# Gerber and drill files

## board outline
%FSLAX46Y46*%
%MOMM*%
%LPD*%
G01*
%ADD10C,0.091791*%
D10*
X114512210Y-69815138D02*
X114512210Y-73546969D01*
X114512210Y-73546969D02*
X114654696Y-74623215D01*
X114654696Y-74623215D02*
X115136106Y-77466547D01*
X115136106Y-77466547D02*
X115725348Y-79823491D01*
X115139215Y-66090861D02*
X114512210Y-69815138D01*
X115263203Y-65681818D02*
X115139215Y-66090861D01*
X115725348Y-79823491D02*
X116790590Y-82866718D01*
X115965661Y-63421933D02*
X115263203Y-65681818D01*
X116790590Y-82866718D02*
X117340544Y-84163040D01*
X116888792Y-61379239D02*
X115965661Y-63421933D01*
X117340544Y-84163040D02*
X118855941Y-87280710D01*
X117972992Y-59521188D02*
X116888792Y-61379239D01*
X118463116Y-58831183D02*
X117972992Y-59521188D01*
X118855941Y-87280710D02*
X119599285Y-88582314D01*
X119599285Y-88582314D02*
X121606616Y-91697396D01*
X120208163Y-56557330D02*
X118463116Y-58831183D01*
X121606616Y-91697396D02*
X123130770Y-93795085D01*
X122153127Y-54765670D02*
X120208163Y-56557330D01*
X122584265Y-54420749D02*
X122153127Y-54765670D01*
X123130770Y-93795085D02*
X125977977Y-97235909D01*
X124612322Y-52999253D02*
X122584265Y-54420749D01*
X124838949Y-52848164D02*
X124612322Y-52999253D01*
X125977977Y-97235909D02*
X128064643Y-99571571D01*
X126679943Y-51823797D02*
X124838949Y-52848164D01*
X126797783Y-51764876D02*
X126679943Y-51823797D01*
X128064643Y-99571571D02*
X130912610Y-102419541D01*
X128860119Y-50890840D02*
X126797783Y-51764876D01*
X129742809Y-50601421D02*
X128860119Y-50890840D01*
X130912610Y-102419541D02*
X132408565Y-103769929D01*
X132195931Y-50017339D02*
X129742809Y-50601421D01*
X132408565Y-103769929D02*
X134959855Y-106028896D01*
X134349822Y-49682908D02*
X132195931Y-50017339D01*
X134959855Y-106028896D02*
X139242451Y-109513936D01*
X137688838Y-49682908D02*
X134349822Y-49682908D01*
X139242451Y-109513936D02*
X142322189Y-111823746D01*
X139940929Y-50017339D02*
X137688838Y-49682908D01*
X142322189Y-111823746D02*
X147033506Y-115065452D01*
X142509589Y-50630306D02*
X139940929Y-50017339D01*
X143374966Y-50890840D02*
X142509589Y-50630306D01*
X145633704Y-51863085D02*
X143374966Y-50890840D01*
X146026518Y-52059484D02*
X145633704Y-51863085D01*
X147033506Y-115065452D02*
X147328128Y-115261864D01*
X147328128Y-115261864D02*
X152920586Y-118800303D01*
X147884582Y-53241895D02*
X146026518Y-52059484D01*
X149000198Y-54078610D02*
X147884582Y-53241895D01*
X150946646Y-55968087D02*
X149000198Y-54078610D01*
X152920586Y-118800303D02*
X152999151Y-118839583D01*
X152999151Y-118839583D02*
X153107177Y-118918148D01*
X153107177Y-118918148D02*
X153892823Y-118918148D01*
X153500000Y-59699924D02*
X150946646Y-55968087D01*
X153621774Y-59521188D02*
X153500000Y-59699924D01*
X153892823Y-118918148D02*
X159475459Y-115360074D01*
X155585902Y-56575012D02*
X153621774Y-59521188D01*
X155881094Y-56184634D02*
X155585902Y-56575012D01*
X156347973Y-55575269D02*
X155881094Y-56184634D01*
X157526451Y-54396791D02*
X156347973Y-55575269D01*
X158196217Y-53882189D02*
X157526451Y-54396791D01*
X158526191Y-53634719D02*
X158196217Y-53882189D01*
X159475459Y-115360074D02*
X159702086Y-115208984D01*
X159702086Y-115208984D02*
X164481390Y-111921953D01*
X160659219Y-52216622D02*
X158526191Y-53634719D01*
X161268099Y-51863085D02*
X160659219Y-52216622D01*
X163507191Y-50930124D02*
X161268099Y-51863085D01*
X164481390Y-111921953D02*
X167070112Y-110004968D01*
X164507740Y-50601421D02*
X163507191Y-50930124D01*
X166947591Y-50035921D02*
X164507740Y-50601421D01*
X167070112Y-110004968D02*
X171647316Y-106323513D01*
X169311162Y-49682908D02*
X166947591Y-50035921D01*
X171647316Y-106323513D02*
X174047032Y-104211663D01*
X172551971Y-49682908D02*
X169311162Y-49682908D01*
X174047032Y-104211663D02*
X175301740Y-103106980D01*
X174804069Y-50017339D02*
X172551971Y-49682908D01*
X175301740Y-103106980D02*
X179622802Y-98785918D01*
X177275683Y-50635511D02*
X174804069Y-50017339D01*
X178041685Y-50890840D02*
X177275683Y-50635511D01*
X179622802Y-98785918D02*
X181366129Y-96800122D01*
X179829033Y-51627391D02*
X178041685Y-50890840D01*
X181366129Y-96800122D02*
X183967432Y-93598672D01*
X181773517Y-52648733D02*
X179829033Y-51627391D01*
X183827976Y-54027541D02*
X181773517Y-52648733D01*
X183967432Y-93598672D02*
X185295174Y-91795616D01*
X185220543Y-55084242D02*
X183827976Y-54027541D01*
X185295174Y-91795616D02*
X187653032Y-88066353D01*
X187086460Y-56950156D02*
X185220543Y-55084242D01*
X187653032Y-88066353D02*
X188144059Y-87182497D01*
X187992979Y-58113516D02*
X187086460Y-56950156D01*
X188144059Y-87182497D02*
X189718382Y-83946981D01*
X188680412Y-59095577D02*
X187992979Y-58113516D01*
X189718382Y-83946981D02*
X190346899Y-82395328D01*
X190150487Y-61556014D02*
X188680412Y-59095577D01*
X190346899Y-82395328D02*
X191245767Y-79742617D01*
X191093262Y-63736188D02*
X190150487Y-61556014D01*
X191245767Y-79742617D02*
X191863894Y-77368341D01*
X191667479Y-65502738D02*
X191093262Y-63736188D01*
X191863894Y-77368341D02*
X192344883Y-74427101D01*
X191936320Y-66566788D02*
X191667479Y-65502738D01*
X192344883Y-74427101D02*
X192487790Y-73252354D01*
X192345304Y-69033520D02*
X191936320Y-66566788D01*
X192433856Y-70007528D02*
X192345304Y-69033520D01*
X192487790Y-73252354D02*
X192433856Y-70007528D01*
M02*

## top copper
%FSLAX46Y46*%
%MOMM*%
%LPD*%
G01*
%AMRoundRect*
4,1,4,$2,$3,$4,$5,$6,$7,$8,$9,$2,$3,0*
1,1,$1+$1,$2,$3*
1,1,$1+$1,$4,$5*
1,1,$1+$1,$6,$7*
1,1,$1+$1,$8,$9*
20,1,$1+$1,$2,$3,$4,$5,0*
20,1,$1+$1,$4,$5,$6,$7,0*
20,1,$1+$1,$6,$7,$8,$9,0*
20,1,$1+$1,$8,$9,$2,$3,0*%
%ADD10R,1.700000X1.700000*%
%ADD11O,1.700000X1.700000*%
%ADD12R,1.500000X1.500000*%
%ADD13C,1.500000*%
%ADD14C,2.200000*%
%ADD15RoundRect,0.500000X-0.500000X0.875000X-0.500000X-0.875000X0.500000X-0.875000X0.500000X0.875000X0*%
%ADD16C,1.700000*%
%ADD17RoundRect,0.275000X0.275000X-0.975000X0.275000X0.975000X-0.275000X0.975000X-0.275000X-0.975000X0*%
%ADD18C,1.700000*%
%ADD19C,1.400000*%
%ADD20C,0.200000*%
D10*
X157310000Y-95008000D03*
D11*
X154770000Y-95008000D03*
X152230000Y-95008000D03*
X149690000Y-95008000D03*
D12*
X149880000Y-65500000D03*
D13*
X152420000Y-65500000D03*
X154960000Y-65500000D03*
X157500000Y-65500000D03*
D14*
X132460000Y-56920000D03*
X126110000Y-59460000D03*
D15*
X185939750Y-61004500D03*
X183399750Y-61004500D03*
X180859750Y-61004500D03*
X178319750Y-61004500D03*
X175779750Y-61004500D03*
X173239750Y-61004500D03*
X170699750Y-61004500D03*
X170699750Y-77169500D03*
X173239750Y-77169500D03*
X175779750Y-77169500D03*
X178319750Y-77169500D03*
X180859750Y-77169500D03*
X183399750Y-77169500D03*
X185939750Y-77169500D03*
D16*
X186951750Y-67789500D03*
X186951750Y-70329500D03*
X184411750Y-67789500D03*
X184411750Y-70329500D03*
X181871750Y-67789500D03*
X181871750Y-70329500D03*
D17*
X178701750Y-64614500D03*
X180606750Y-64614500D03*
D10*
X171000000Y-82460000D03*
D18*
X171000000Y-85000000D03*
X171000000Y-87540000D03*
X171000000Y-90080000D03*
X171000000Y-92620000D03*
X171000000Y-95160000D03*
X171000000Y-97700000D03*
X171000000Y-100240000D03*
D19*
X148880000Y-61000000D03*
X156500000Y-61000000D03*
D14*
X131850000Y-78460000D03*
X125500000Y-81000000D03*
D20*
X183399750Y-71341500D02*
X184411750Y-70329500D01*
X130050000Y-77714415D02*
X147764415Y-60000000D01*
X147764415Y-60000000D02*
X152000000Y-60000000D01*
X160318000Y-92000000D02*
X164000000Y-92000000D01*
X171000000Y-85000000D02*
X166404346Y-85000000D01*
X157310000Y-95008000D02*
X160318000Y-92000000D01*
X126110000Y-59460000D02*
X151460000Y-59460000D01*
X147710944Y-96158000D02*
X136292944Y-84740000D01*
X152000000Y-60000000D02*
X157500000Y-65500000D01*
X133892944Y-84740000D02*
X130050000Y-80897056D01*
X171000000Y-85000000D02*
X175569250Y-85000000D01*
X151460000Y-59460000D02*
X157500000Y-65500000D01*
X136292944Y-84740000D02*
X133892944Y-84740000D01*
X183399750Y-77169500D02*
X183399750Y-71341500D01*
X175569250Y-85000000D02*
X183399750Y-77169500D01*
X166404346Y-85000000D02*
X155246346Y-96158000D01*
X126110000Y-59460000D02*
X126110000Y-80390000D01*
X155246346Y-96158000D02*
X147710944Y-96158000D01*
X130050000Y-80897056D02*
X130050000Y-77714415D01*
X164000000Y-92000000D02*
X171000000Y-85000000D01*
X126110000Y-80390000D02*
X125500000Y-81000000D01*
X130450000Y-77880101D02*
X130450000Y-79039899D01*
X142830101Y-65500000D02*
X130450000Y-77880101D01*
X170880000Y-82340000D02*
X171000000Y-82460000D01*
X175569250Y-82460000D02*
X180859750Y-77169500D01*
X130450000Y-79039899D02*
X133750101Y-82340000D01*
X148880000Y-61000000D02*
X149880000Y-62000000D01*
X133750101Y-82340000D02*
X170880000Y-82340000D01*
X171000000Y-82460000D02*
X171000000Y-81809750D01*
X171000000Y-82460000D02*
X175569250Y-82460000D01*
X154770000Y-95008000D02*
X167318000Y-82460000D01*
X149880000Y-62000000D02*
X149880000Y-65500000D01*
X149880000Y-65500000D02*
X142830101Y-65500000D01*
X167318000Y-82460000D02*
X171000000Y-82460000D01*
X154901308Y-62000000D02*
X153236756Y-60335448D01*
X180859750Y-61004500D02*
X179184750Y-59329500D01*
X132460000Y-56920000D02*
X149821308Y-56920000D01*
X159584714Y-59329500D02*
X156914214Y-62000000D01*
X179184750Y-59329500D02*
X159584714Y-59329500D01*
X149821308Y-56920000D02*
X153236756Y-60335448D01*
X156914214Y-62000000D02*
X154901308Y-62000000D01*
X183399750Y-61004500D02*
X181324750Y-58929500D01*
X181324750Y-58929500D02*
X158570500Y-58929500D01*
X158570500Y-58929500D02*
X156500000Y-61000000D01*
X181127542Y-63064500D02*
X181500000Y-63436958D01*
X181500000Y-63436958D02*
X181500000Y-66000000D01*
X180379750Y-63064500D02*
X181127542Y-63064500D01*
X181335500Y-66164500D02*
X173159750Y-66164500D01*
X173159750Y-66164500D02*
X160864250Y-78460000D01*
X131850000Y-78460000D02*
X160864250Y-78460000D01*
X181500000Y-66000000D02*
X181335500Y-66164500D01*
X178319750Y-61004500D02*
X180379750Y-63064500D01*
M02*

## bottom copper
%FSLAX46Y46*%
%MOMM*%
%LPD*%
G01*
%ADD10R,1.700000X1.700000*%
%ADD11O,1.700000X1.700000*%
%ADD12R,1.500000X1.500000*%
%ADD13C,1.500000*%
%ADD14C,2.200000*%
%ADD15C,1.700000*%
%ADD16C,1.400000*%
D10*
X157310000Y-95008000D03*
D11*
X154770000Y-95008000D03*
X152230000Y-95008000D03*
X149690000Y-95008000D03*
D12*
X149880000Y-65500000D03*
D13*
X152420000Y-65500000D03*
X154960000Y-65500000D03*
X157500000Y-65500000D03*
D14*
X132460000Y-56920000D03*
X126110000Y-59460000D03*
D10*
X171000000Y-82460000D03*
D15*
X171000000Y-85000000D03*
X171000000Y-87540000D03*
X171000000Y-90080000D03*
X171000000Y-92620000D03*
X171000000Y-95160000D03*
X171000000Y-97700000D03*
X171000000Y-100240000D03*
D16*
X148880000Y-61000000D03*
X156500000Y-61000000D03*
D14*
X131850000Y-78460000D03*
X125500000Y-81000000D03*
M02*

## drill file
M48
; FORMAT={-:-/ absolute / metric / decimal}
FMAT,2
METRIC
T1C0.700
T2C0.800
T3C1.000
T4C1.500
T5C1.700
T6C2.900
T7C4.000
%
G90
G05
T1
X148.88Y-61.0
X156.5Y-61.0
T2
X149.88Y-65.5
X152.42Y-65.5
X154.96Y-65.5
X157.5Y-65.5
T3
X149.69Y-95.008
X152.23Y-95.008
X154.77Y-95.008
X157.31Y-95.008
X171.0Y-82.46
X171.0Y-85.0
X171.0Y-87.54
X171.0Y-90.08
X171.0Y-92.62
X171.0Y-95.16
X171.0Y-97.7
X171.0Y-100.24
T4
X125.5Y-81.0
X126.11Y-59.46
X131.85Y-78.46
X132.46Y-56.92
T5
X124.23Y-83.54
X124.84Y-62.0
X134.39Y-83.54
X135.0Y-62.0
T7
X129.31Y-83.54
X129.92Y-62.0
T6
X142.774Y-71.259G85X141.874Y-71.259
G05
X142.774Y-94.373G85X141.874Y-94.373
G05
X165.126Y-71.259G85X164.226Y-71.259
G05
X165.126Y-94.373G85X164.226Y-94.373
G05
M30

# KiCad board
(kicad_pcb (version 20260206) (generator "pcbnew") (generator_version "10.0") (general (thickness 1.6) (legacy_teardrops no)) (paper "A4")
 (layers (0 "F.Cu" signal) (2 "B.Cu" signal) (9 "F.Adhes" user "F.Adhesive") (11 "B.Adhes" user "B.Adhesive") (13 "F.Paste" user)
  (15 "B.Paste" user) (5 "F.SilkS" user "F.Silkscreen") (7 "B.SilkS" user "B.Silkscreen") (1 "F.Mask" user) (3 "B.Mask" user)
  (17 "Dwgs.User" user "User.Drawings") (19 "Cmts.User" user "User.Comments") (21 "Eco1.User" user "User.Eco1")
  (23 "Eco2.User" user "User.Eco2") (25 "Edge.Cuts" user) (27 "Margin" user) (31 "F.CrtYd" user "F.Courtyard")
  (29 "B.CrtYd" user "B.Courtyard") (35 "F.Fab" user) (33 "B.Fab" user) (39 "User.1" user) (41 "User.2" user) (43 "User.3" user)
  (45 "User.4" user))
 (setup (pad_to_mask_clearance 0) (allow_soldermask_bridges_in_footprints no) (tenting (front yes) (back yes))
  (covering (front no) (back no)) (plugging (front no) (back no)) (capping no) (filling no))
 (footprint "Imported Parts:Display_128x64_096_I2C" (layer "F.Cu") (at 153.5 95.008 180)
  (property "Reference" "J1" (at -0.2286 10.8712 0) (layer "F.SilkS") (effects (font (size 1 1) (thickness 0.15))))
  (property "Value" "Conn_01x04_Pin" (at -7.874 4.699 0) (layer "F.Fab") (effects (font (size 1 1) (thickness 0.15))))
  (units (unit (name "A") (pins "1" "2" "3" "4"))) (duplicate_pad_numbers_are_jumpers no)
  (pad "" np_thru_hole oval (at -11.176 0.635 180) (size 3.8 2.9) (drill oval 3.8 2.9) (layers "*.Cu" "*.Mask"))
  (pad "" np_thru_hole oval (at -11.176 23.749 180) (size 3.8 2.9) (drill oval 3.8 2.9) (layers "*.Cu" "*.Mask"))
  (pad "" np_thru_hole oval (at 11.176 0.635 180) (size 3.8 2.9) (drill oval 3.8 2.9) (layers "*.Cu" "*.Mask"))
  (pad "" np_thru_hole oval (at 11.176 23.749 180) (size 3.8 2.9) (drill oval 3.8 2.9) (layers "*.Cu" "*.Mask"))
  (pad "1" thru_hole rect (at -3.81 0 270) (size 1.7 1.7) (drill 1) (layers "*.Cu" "*.Mask") (remove_unused_layers no) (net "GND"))
  (pad "2" thru_hole oval (at -1.27 0 270) (size 1.7 1.7) (drill 1) (layers "*.Cu" "*.Mask") (remove_unused_layers no) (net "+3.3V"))
  (pad "3" thru_hole oval (at 1.27 0 270) (size 1.7 1.7) (drill 1) (layers "*.Cu" "*.Mask") (remove_unused_layers no)
   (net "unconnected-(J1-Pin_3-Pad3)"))
  (pad "4" thru_hole oval (at 3.81 0 270) (size 1.7 1.7) (drill 1) (layers "*.Cu" "*.Mask") (remove_unused_layers no)
   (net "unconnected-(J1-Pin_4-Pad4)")))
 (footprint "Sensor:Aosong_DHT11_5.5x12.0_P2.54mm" (layer "F.Cu") (at 149.88 65.5 90)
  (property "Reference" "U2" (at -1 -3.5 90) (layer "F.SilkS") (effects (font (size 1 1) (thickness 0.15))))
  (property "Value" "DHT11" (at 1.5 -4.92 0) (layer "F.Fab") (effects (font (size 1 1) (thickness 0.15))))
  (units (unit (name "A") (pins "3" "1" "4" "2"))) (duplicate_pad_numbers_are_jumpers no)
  (pad "1" thru_hole rect (at 0 0 90) (size 1.5 1.5) (drill 0.8) (layers "*.Cu" "*.Mask") (remove_unused_layers no) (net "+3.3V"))
  (pad "2" thru_hole circle (at 0 2.54 90) (size 1.5 1.5) (drill 0.8) (layers "*.Cu" "*.Mask") (remove_unused_layers no)
   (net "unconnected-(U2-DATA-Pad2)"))
  (pad "3" thru_hole circle (at 0 5.08 90) (size 1.5 1.5) (drill 0.8) (layers "*.Cu" "*.Mask") (remove_unused_layers no)
   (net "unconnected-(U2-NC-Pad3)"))
  (pad "4" thru_hole circle (at 0 7.62 90) (size 1.5 1.5) (drill 0.8) (layers "*.Cu" "*.Mask") (remove_unused_layers no) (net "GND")))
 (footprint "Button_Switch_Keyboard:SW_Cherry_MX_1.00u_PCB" (layer "F.Cu") (at 132.46 56.92)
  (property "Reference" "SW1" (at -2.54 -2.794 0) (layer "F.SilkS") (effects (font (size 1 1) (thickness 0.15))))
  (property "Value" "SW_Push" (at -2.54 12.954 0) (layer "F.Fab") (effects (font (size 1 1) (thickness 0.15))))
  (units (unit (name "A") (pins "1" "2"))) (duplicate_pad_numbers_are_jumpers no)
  (pad "" np_thru_hole circle (at -7.62 5.08) (size 1.7 1.7) (drill 1.7) (layers "*.Cu" "*.Mask"))
  (pad "" np_thru_hole circle (at -2.54 5.08) (size 4 4) (drill 4) (layers "*.Cu" "*.Mask"))
  (pad "" np_thru_hole circle (at 2.54 5.08) (size 1.7 1.7) (drill 1.7) (layers "*.Cu" "*.Mask"))
  (pad "1" thru_hole circle (at 0 0) (size 2.2 2.2) (drill 1.5) (layers "*.Cu" "*.Mask") (remove_unused_layers no) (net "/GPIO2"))
  (pad "2" thru_hole circle (at -6.35 2.54) (size 2.2 2.2) (drill 1.5) (layers "*.Cu" "*.Mask") (remove_unused_layers no) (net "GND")))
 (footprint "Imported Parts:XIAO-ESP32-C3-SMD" (layer "F.Cu") (at 167.81975 60.1695 -90)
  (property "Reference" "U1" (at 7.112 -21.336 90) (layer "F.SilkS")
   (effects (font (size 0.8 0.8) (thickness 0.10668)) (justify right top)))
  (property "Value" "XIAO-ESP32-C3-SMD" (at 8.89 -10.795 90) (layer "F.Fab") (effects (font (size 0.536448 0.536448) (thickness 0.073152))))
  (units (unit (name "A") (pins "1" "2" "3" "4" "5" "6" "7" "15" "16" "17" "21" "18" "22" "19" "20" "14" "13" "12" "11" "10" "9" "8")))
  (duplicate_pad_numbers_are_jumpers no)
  (pad "1" smd roundrect (at 0.835 -18.12 270) (size 2.75 2) (layers "F.Cu" "F.Mask" "F.Paste") (roundrect_rratio 0.25)
   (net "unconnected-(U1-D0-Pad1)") (solder_mask_margin 0.0508) (thermal_bridge_angle 45))
  (pad "2" smd roundrect (at 0.835 -15.58 270) (size 2.75 2) (layers "F.Cu" "F.Mask" "F.Paste") (roundrect_rratio 0.25) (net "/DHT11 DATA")
   (solder_mask_margin 0.0508) (thermal_bridge_angle 45))
  (pad "3" smd roundrect (at 0.835 -13.04 270) (size 2.75 2) (layers "F.Cu" "F.Mask" "F.Paste") (roundrect_rratio 0.25) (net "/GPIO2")
   (solder_mask_margin 0.0508) (thermal_bridge_angle 45))
  (pad "4" smd roundrect (at 0.835 -10.5 270) (size 2.75 2) (layers "F.Cu" "F.Mask" "F.Paste") (roundrect_rratio 0.25) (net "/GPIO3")
   (solder_mask_margin 0.0508) (thermal_bridge_angle 45))
  (pad "5" smd roundrect (at 0.835 -7.96 270) (size 2.75 2) (layers "F.Cu" "F.Mask" "F.Paste") (roundrect_rratio 0.25) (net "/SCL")
   (solder_mask_margin 0.0508) (thermal_bridge_angle 45))
  (pad "6" smd roundrect (at 0.835 -5.42 270) (size 2.75 2) (layers "F.Cu" "F.Mask" "F.Paste") (roundrect_rratio 0.25) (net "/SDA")
   (solder_mask_margin 0.0508) (thermal_bridge_angle 45))
  (pad "7" smd roundrect (at 0.835 -2.88 270) (size 2.75 2) (layers "F.Cu" "F.Mask" "F.Paste") (roundrect_rratio 0.25)
   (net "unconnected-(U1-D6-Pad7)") (solder_mask_margin 0.0508) (thermal_bridge_angle 45))
  (pad "8" smd roundrect (at 17 -2.88 270) (size 2.75 2) (layers "F.Cu" "F.Mask" "F.Paste") (roundrect_rratio 0.25)
   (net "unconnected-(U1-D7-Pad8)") (solder_mask_margin 0.0508) (thermal_bridge_angle 45))
  (pad "9" smd roundrect (at 17 -5.42 270) (size 2.75 2) (layers "F.Cu" "F.Mask" "F.Paste") (roundrect_rratio 0.25)
   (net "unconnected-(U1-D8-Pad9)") (solder_mask_margin 0.0508) (thermal_bridge_angle 45))
  (pad "10" smd roundrect (at 17 -7.96 270) (size 2.75 2) (layers "F.Cu" "F.Mask" "F.Paste") (roundrect_rratio 0.25)
   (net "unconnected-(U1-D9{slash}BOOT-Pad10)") (solder_mask_margin 0.0508) (thermal_bridge_angle 45))
  (pad "11" smd roundrect (at 17 -10.5 270) (size 2.75 2) (layers "F.Cu" "F.Mask" "F.Paste") (roundrect_rratio 0.25)
   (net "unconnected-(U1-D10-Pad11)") (solder_mask_margin 0.0508) (thermal_bridge_angle 45))
  (pad "12" smd roundrect (at 17 -13.04 270) (size 2.75 2) (layers "F.Cu" "F.Mask" "F.Paste") (roundrect_rratio 0.25) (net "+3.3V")
   (solder_mask_margin 0.0508) (thermal_bridge_angle 45))
  (pad "13" smd roundrect (at 17 -15.58 270) (size 2.75 2) (layers "F.Cu" "F.Mask" "F.Paste") (roundrect_rratio 0.25) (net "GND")
   (solder_mask_margin 0.0508) (thermal_bridge_angle 45))
  (pad "14" smd roundrect (at 17 -18.12 270) (size 2.75 2) (layers "F.Cu" "F.Mask" "F.Paste") (roundrect_rratio 0.25) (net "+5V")
   (solder_mask_margin 0.0508) (thermal_bridge_angle 45))
  (pad "15" smd circle (at 7.62 -19.132 270) (size 1.7 1.7) (layers "F.Cu" "F.Mask" "F.Paste") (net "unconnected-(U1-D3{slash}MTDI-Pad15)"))
  (pad "16" smd circle (at 10.16 -19.132 270) (size 1.7 1.7) (layers "F.Cu" "F.Mask" "F.Paste") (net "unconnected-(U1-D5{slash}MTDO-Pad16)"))
  (pad "17" smd circle (at 7.62 -16.592 270) (size 1.7 1.7) (layers "F.Cu" "F.Mask" "F.Paste") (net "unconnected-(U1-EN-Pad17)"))
  (pad "18" smd circle (at 10.16 -16.592 270) (size 1.7 1.7) (layers "F.Cu" "F.Mask" "F.Paste") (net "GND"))
  (pad "19" smd circle (at 7.62 -14.052 270) (size 1.7 1.7) (layers "F.Cu" "F.Mask" "F.Paste") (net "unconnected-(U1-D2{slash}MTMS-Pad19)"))
  (pad "20" smd circle (at 10.16 -14.052 270) (size 1.7 1.7) (layers "F.Cu" "F.Mask" "F.Paste") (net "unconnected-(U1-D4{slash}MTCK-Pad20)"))
  (pad "21" smd roundrect (at 4.445 -10.882 90) (size 2.5 1.1) (layers "F.Cu" "F.Mask" "F.Paste") (roundrect_rratio 0.25)
   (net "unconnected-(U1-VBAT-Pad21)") (thermal_bridge_angle 45))
  (pad "22" smd roundrect (at 4.445 -12.787 90) (size 2.5 1.1) (layers "F.Cu" "F.Mask" "F.Paste") (roundrect_rratio 0.25)
   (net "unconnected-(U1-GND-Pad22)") (thermal_bridge_angle 45)))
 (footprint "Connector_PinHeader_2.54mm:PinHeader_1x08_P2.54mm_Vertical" (layer "F.Cu") (at 171 82.46)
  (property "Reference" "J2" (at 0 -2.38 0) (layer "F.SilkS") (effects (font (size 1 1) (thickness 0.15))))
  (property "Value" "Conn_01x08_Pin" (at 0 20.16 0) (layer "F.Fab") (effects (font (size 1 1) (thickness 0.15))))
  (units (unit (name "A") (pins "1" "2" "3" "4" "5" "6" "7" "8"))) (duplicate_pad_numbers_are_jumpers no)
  (pad "1" thru_hole rect (at 0 0) (size 1.7 1.7) (drill 1) (layers "*.Cu" "*.Mask") (remove_unused_layers no) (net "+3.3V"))
  (pad "2" thru_hole circle (at 0 2.54) (size 1.7 1.7) (drill 1) (layers "*.Cu" "*.Mask") (remove_unused_layers no) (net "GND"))
  (pad "3" thru_hole circle (at 0 5.08) (size 1.7 1.7) (drill 1) (layers "*.Cu" "*.Mask") (remove_unused_layers no)
   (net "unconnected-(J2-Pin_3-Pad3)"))
  (pad "4" thru_hole circle (at 0 7.62) (size 1.7 1.7) (drill 1) (layers "*.Cu" "*.Mask") (remove_unused_layers no)
   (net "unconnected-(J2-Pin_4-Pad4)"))
  (pad "5" thru_hole circle (at 0 10.16) (size 1.7 1.7) (drill 1) (layers "*.Cu" "*.Mask") (remove_unused_layers no)
   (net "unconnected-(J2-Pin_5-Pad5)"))
  (pad "6" thru_hole circle (at 0 12.7) (size 1.7 1.7) (drill 1) (layers "*.Cu" "*.Mask") (remove_unused_layers no)
   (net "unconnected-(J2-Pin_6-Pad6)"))
  (pad "7" thru_hole circle (at 0 15.24) (size 1.7 1.7) (drill 1) (layers "*.Cu" "*.Mask") (remove_unused_layers no)
   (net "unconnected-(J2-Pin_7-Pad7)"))
  (pad "8" thru_hole circle (at 0 17.78) (size 1.7 1.7) (drill 1) (layers "*.Cu" "*.Mask") (remove_unused_layers no)
   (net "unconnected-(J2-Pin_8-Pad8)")))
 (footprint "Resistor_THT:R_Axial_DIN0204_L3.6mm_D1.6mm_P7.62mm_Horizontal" (layer "F.Cu") (at 148.88 61)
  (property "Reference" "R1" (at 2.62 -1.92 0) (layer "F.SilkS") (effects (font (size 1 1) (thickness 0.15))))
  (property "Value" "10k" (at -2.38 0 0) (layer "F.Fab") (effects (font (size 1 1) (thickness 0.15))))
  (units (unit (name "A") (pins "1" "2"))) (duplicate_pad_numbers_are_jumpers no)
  (pad "1" thru_hole circle (at 0 0) (size 1.4 1.4) (drill 0.7) (layers "*.Cu" "*.Mask") (remove_unused_layers no) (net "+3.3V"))
  (pad "2" thru_hole circle (at 7.62 0) (size 1.4 1.4) (drill 0.7) (layers "*.Cu" "*.Mask") (remove_unused_layers no) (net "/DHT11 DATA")))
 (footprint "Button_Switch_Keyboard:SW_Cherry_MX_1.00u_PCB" (layer "F.Cu") (at 131.85 78.46)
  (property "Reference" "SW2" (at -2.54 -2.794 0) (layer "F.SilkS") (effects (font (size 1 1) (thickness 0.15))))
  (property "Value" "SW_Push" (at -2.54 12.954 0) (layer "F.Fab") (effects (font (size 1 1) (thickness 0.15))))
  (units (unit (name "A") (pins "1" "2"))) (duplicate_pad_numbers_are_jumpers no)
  (pad "" np_thru_hole circle (at -7.62 5.08) (size 1.7 1.7) (drill 1.7) (layers "*.Cu" "*.Mask"))
  (pad "" np_thru_hole circle (at -2.54 5.08) (size 4 4) (drill 4) (layers "*.Cu" "*.Mask"))
  (pad "" np_thru_hole circle (at 2.54 5.08) (size 1.7 1.7) (drill 1.7) (layers "*.Cu" "*.Mask"))
  (pad "1" thru_hole circle (at 0 0) (size 2.2 2.2) (drill 1.5) (layers "*.Cu" "*.Mask") (remove_unused_layers no) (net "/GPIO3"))
  (pad "2" thru_hole circle (at -6.35 2.54) (size 2.2 2.2) (drill 1.5) (layers "*.Cu" "*.Mask") (remove_unused_layers no) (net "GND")))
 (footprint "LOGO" (layer "F.Cu") (at 154.5 106)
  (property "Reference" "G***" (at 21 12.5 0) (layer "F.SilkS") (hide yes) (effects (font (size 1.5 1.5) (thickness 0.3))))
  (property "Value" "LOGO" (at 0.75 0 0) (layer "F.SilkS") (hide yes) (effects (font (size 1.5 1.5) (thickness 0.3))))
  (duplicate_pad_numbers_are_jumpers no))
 (gr_line (start 114.51221 69.815138) (end 114.51221 73.546969) (stroke (width 0.091791) (type default)) (locked yes) (layer "Edge.Cuts"))
 (gr_line (start 114.51221 73.546969) (end 114.654696 74.623215) (stroke (width 0.091791) (type default)) (locked yes) (layer "Edge.Cuts"))
 (gr_line (start 114.654696 74.623215) (end 115.136106 77.466547) (stroke (width 0.091791) (type default)) (locked yes) (layer "Edge.Cuts"))
 (gr_line (start 115.136106 77.466547) (end 115.725348 79.823491) (stroke (width 0.091791) (type default)) (locked yes) (layer "Edge.Cuts"))
 (gr_line (start 115.139215 66.090861) (end 114.51221 69.815138) (stroke (width 0.091791) (type default)) (locked yes) (layer "Edge.Cuts"))
 (gr_line (start 115.263203 65.681818) (end 115.139215 66.090861) (stroke (width 0.091791) (type default)) (locked yes) (layer "Edge.Cuts"))
 (gr_line (start 115.725348 79.823491) (end 116.79059 82.866718) (stroke (width 0.091791) (type default)) (locked yes) (layer "Edge.Cuts"))
 (gr_line (start 115.965661 63.421933) (end 115.263203 65.681818) (stroke (width 0.091791) (type default)) (locked yes) (layer "Edge.Cuts"))
 (gr_line (start 116.79059 82.866718) (end 117.340544 84.16304) (stroke (width 0.091791) (type default)) (locked yes) (layer "Edge.Cuts"))
 (gr_line (start 116.888792 61.379239) (end 115.965661 63.421933) (stroke (width 0.091791) (type default)) (locked yes) (layer "Edge.Cuts"))
 (gr_line (start 117.340544 84.16304) (end 118.855941 87.28071) (stroke (width 0.091791) (type default)) (locked yes) (layer "Edge.Cuts"))
 (gr_line (start 117.972992 59.521188) (end 116.888792 61.379239) (stroke (width 0.091791) (type default)) (locked yes) (layer "Edge.Cuts"))
 (gr_line (start 118.463116 58.831183) (end 117.972992 59.521188) (stroke (width 0.091791) (type default)) (locked yes) (layer "Edge.Cuts"))
 (gr_line (start 118.855941 87.28071) (end 119.599285 88.582314) (stroke (width 0.091791) (type default)) (locked yes) (layer "Edge.Cuts"))
 (gr_line (start 119.599285 88.582314) (end 121.606616 91.697396) (stroke (width 0.091791) (type default)) (locked yes) (layer "Edge.Cuts"))
 (gr_line (start 120.208163 56.55733) (end 118.463116 58.831183) (stroke (width 0.091791) (type default)) (locked yes) (layer "Edge.Cuts"))
 (gr_line (start 121.606616 91.697396) (end 123.13077 93.795085) (stroke (width 0.091791) (type default)) (locked yes) (layer "Edge.Cuts"))
 (gr_line (start 122.153127 54.76567) (end 120.208163 56.55733) (stroke (width 0.091791) (type default)) (locked yes) (layer "Edge.Cuts"))
 (gr_line (start 122.584265 54.420749) (end 122.153127 54.76567) (stroke (width 0.091791) (type default)) (locked yes) (layer "Edge.Cuts"))
 (gr_line (start 123.13077 93.795085) (end 125.977977 97.235909) (stroke (width 0.091791) (type default)) (locked yes) (layer "Edge.Cuts"))
 (gr_line (start 124.612322 52.999253) (end 122.584265 54.420749) (stroke (width 0.091791) (type default)) (locked yes) (layer "Edge.Cuts"))
 (gr_line (start 124.838949 52.848164) (end 124.612322 52.999253) (stroke (width 0.091791) (type default)) (locked yes) (layer "Edge.Cuts"))
 (gr_line (start 125.977977 97.235909) (end 128.064643 99.571571) (stroke (width 0.091791) (type default)) (locked yes) (layer "Edge.Cuts"))
 (gr_line (start 126.679943 51.823797) (end 124.838949 52.848164) (stroke (width 0.091791) (type default)) (locked yes) (layer "Edge.Cuts"))
 (gr_line (start 126.797783 51.764876) (end 126.679943 51.823797) (stroke (width 0.091791) (type default)) (locked yes) (layer "Edge.Cuts"))
 (gr_line (start 128.064643 99.571571) (end 130.91261 102.419541) (stroke (width 0.091791) (type default)) (locked yes) (layer "Edge.Cuts"))
 (gr_line (start 128.860119 50.89084) (end 126.797783 51.764876) (stroke (width 0.091791) (type default)) (locked yes) (layer "Edge.Cuts"))
 (gr_line (start 129.742809 50.601421) (end 128.860119 50.89084) (stroke (width 0.091791) (type default)) (locked yes) (layer "Edge.Cuts"))
 (gr_line (start 130.91261 102.419541) (end 132.408565 103.769929) (stroke (width 0.091791) (type default)) (locked yes) (layer "Edge.Cuts"))
 (gr_line (start 132.195931 50.017339) (end 129.742809 50.601421) (stroke (width 0.091791) (type default)) (locked yes) (layer "Edge.Cuts"))
 (gr_line (start 132.408565 103.769929) (end 134.959855 106.028896) (stroke (width 0.091791) (type default)) (locked yes)
  (layer "Edge.Cuts"))
 (gr_line (start 134.349822 49.682908) (end 132.195931 50.017339) (stroke (width 0.091791) (type default)) (locked yes) (layer "Edge.Cuts"))
 (gr_line (start 134.959855 106.028896) (end 139.242451 109.513936) (stroke (width 0.091791) (type default)) (locked yes)
  (layer "Edge.Cuts"))
 (gr_line (start 137.688838 49.682908) (end 134.349822 49.682908) (stroke (width 0.091791) (type default)) (locked yes) (layer "Edge.Cuts"))
 (gr_line (start 139.242451 109.513936) (end 142.322189 111.823746) (stroke (width 0.091791) (type default)) (locked yes)
  (layer "Edge.Cuts"))
 (gr_line (start 139.940929 50.017339) (end 137.688838 49.682908) (stroke (width 0.091791) (type default)) (locked yes) (layer "Edge.Cuts"))
 (gr_line (start 142.322189 111.823746) (end 147.033506 115.065452) (stroke (width 0.091791) (type default)) (locked yes)
  (layer "Edge.Cuts"))
 (gr_line (start 142.509589 50.630306) (end 139.940929 50.017339) (stroke (width 0.091791) (type default)) (locked yes) (layer "Edge.Cuts"))
 (gr_line (start 143.374966 50.89084) (end 142.509589 50.630306) (stroke (width 0.091791) (type default)) (locked yes) (layer "Edge.Cuts"))
 (gr_line (start 145.633704 51.863085) (end 143.374966 50.89084) (stroke (width 0.091791) (type default)) (locked yes) (layer "Edge.Cuts"))
 (gr_line (start 146.026518 52.059484) (end 145.633704 51.863085) (stroke (width 0.091791) (type default)) (locked yes) (layer "Edge.Cuts"))
 (gr_line (start 147.033506 115.065452) (end 147.328128 115.261864) (stroke (width 0.091791) (type default)) (locked yes)
  (layer "Edge.Cuts"))
 (gr_line (start 147.328128 115.261864) (end 152.920586 118.800303) (stroke (width 0.091791) (type default)) (locked yes)
  (layer "Edge.Cuts"))
 (gr_line (start 147.884582 53.241895) (end 146.026518 52.059484) (stroke (width 0.091791) (type default)) (locked yes) (layer "Edge.Cuts"))
 (gr_line (start 149.000198 54.07861) (end 147.884582 53.241895) (stroke (width 0.091791) (type default)) (locked yes) (layer "Edge.Cuts"))
 (gr_line (start 150.946646 55.968087) (end 149.000198 54.07861) (stroke (width 0.091791) (type default)) (locked yes) (layer "Edge.Cuts"))
 (gr_line (start 152.920586 118.800303) (end 152.999151 118.839583) (stroke (width 0.091791) (type default)) (locked yes)
  (layer "Edge.Cuts"))
 (gr_line (start 152.999151 118.839583) (end 153.107177 118.918148) (stroke (width 0.091791) (type default)) (locked yes)
  (layer "Edge.Cuts"))
 (gr_line (start 153.107177 118.918148) (end 153.892823 118.918148) (stroke (width 0.091791) (type default)) (locked yes)
  (layer "Edge.Cuts"))
 (gr_line (start 153.5 59.699924) (end 150.946646 55.968087) (stroke (width 0.091791) (type default)) (locked yes) (layer "Edge.Cuts"))
 (gr_line (start 153.621774 59.521188) (end 153.5 59.699924) (stroke (width 0.091791) (type default)) (locked yes) (layer "Edge.Cuts"))
 (gr_line (start 153.892823 118.918148) (end 159.475459 115.360074) (stroke (width 0.091791) (type default)) (locked yes)
  (layer "Edge.Cuts"))
 (gr_line (start 155.585902 56.575012) (end 153.621774 59.521188) (stroke (width 0.091791) (type default)) (locked yes) (layer "Edge.Cuts"))
 (gr_line (start 155.881094 56.184634) (end 155.585902 56.575012) (stroke (width 0.091791) (type default)) (locked yes) (layer "Edge.Cuts"))
 (gr_line (start 156.347973 55.575269) (end 155.881094 56.184634) (stroke (width 0.091791) (type default)) (locked yes) (layer "Edge.Cuts"))
 (gr_line (start 157.526451 54.396791) (end 156.347973 55.575269) (stroke (width 0.091791) (type default)) (locked yes) (layer "Edge.Cuts"))
 (gr_line (start 158.196217 53.882189) (end 157.526451 54.396791) (stroke (width 0.091791) (type default)) (locked yes) (layer "Edge.Cuts"))
 (gr_line (start 158.526191 53.634719) (end 158.196217 53.882189) (stroke (width 0.091791) (type default)) (locked yes) (layer "Edge.Cuts"))
 (gr_line (start 159.475459 115.360074) (end 159.702086 115.208984) (stroke (width 0.091791) (type default)) (locked yes)
  (layer "Edge.Cuts"))
 (gr_line (start 159.702086 115.208984) (end 164.48139 111.921953) (stroke (width 0.091791) (type default)) (locked yes) (layer "Edge.Cuts"))
 (gr_line (start 160.659219 52.216622) (end 158.526191 53.634719) (stroke (width 0.091791) (type default)) (locked yes) (layer "Edge.Cuts"))
 (gr_line (start 161.268099 51.863085) (end 160.659219 52.216622) (stroke (width 0.091791) (type default)) (locked yes) (layer "Edge.Cuts"))
 (gr_line (start 163.507191 50.930124) (end 161.268099 51.863085) (stroke (width 0.091791) (type default)) (locked yes) (layer "Edge.Cuts"))
 (gr_line (start 164.48139 111.921953) (end 167.070112 110.004968) (stroke (width 0.091791) (type default)) (locked yes) (layer "Edge.Cuts"))
 (gr_line (start 164.50774 50.601421) (end 163.507191 50.930124) (stroke (width 0.091791) (type default)) (locked yes) (layer "Edge.Cuts"))
 (gr_line (start 166.947591 50.035921) (end 164.50774 50.601421) (stroke (width 0.091791) (type default)) (locked yes) (layer "Edge.Cuts"))
 (gr_line (start 167.070112 110.004968) (end 171.647316 106.323513) (stroke (width 0.091791) (type default)) (locked yes)
  (layer "Edge.Cuts"))
 (gr_line (start 169.311162 49.682908) (end 166.947591 50.035921) (stroke (width 0.091791) (type default)) (locked yes) (layer "Edge.Cuts"))
 (gr_line (start 171.647316 106.323513) (end 174.047032 104.211663) (stroke (width 0.091791) (type default)) (locked yes)
  (layer "Edge.Cuts"))
 (gr_line (start 172.551971 49.682908) (end 169.311162 49.682908) (stroke (width 0.091791) (type default)) (locked yes) (layer "Edge.Cuts"))
 (gr_line (start 174.047032 104.211663) (end 175.30174 103.10698) (stroke (width 0.091791) (type default)) (locked yes) (layer "Edge.Cuts"))
 (gr_line (start 174.804069 50.017339) (end 172.551971 49.682908) (stroke (width 0.091791) (type default)) (locked yes) (layer "Edge.Cuts"))
 (gr_line (start 175.30174 103.10698) (end 179.622802 98.785918) (stroke (width 0.091791) (type default)) (locked yes) (layer "Edge.Cuts"))
 (gr_line (start 177.275683 50.635511) (end 174.804069 50.017339) (stroke (width 0.091791) (type default)) (locked yes) (layer "Edge.Cuts"))
 (gr_line (start 178.041685 50.89084) (end 177.275683 50.635511) (stroke (width 0.091791) (type default)) (locked yes) (layer "Edge.Cuts"))
 (gr_line (start 179.622802 98.785918) (end 181.366129 96.800122) (stroke (width 0.091791) (type default)) (locked yes) (layer "Edge.Cuts"))
 (gr_line (start 179.829033 51.627391) (end 178.041685 50.89084) (stroke (width 0.091791) (type default)) (locked yes) (layer "Edge.Cuts"))
 (gr_line (start 181.366129 96.800122) (end 183.967432 93.598672) (stroke (width 0.091791) (type default)) (locked yes) (layer "Edge.Cuts"))
 (gr_line (start 181.773517 52.648733) (end 179.829033 51.627391) (stroke (width 0.091791) (type default)) (locked yes) (layer "Edge.Cuts"))
 (gr_line (start 183.827976 54.027541) (end 181.773517 52.648733) (stroke (width 0.091791) (type default)) (locked yes) (layer "Edge.Cuts"))
 (gr_line (start 183.967432 93.598672) (end 185.295174 91.795616) (stroke (width 0.091791) (type default)) (locked yes) (layer "Edge.Cuts"))
 (gr_line (start 185.220543 55.084242) (end 183.827976 54.027541) (stroke (width 0.091791) (type default)) (locked yes) (layer "Edge.Cuts"))
 (gr_line (start 185.295174 91.795616) (end 187.653032 88.066353) (stroke (width 0.091791) (type default)) (locked yes) (layer "Edge.Cuts"))
 (gr_line (start 187.08646 56.950156) (end 185.220543 55.084242) (stroke (width 0.091791) (type default)) (locked yes) (layer "Edge.Cuts"))
 (gr_line (start 187.653032 88.066353) (end 188.144059 87.182497) (stroke (width 0.091791) (type default)) (locked yes) (layer "Edge.Cuts"))
 (gr_line (start 187.992979 58.113516) (end 187.08646 56.950156) (stroke (width 0.091791) (type default)) (locked yes) (layer "Edge.Cuts"))
 (gr_line (start 188.144059 87.182497) (end 189.718382 83.946981) (stroke (width 0.091791) (type default)) (locked yes) (layer "Edge.Cuts"))
 (gr_line (start 188.680412 59.095577) (end 187.992979 58.113516) (stroke (width 0.091791) (type default)) (locked yes) (layer "Edge.Cuts"))
 (gr_line (start 189.718382 83.946981) (end 190.346899 82.395328) (stroke (width 0.091791) (type default)) (locked yes) (layer "Edge.Cuts"))
 (gr_line (start 190.150487 61.556014) (end 188.680412 59.095577) (stroke (width 0.091791) (type default)) (locked yes) (layer "Edge.Cuts"))
 (gr_line (start 190.346899 82.395328) (end 191.245767 79.742617) (stroke (width 0.091791) (type default)) (locked yes) (layer "Edge.Cuts"))
 (gr_line (start 191.093262 63.736188) (end 190.150487 61.556014) (stroke (width 0.091791) (type default)) (locked yes) (layer "Edge.Cuts"))
 (gr_line (start 191.245767 79.742617) (end 191.863894 77.368341) (stroke (width 0.091791) (type default)) (locked yes) (layer "Edge.Cuts"))
 (gr_line (start 191.667479 65.502738) (end 191.093262 63.736188) (stroke (width 0.091791) (type default)) (locked yes) (layer "Edge.Cuts"))
 (gr_line (start 191.863894 77.368341) (end 192.344883 74.427101) (stroke (width 0.091791) (type default)) (locked yes) (layer "Edge.Cuts"))
 (gr_line (start 191.93632 66.566788) (end 191.667479 65.502738) (stroke (width 0.091791) (type default)) (locked yes) (layer "Edge.Cuts"))
 (gr_line (start 192.344883 74.427101) (end 192.48779 73.252354) (stroke (width 0.091791) (type default)) (locked yes) (layer "Edge.Cuts"))
 (gr_line (start 192.345304 69.03352) (end 191.93632 66.566788) (stroke (width 0.091791) (type default)) (locked yes) (layer "Edge.Cuts"))
 (gr_line (start 192.433856 70.007528) (end 192.345304 69.03352) (stroke (width 0.091791) (type default)) (locked yes) (layer "Edge.Cuts"))
 (gr_line (start 192.48779 73.252354) (end 192.433856 70.007528) (stroke (width 0.091791) (type default)) (locked yes) (layer "Edge.Cuts"))
 (segment (start 183.39975 71.3415) (end 184.41175 70.3295) (width 0.2) (layer "F.Cu") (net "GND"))
 (segment (start 130.05 77.714415) (end 147.764415 60) (width 0.2) (layer "F.Cu") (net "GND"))
 (segment (start 147.764415 60) (end 152 60) (width 0.2) (layer "F.Cu") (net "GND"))
 (segment (start 160.318 92) (end 164 92) (width 0.2) (layer "F.Cu") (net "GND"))
 (segment (start 171 85) (end 166.404346 85) (width 0.2) (layer "F.Cu") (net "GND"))
 (segment (start 157.31 95.008) (end 160.318 92) (width 0.2) (layer "F.Cu") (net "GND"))
 (segment (start 126.11 59.46) (end 151.46 59.46) (width 0.2) (layer "F.Cu") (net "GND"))
 (segment (start 147.710944 96.158) (end 136.292944 84.74) (width 0.2) (layer "F.Cu") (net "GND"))
 (segment (start 152 60) (end 157.5 65.5) (width 0.2) (layer "F.Cu") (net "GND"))
 (segment (start 133.892944 84.74) (end 130.05 80.897056) (width 0.2) (layer "F.Cu") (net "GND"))
 (segment (start 171 85) (end 175.56925 85) (width 0.2) (layer "F.Cu") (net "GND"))
 (segment (start 151.46 59.46) (end 157.5 65.5) (width 0.2) (layer "F.Cu") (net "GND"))
 (segment (start 136.292944 84.74) (end 133.892944 84.74) (width 0.2) (layer "F.Cu") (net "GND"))
 (segment (start 183.39975 77.1695) (end 183.39975 71.3415) (width 0.2) (layer "F.Cu") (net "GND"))
 (segment (start 175.56925 85) (end 183.39975 77.1695) (width 0.2) (layer "F.Cu") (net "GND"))
 (segment (start 166.404346 85) (end 155.246346 96.158) (width 0.2) (layer "F.Cu") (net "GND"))
 (segment (start 126.11 59.46) (end 126.11 80.39) (width 0.2) (layer "F.Cu") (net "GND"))
 (segment (start 155.246346 96.158) (end 147.710944 96.158) (width 0.2) (layer "F.Cu") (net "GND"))
 (segment (start 130.05 80.897056) (end 130.05 77.714415) (width 0.2) (layer "F.Cu") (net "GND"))
 (segment (start 164 92) (end 171 85) (width 0.2) (layer "F.Cu") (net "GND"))
 (segment (start 126.11 80.39) (end 125.5 81) (width 0.2) (layer "F.Cu") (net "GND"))
 (segment (start 130.45 77.880101) (end 130.45 79.039899) (width 0.2) (layer "F.Cu") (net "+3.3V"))
 (segment (start 142.830101 65.5) (end 130.45 77.880101) (width 0.2) (layer "F.Cu") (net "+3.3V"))
 (segment (start 170.88 82.34) (end 171 82.46) (width 0.2) (layer "F.Cu") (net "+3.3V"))
 (segment (start 175.56925 82.46) (end 180.85975 77.1695) (width 0.2) (layer "F.Cu") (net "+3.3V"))
 (segment (start 130.45 79.039899) (end 133.750101 82.34) (width 0.2) (layer "F.Cu") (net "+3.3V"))
 (segment (start 148.88 61) (end 149.88 62) (width 0.2) (layer "F.Cu") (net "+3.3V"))
 (segment (start 133.750101 82.34) (end 170.88 82.34) (width 0.2) (layer "F.Cu") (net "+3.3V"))
 (segment (start 171 82.46) (end 171 81.80975) (width 0.2) (layer "F.Cu") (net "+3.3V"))
 (segment (start 171 82.46) (end 175.56925 82.46) (width 0.2) (layer "F.Cu") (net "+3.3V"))
 (segment (start 154.77 95.008) (end 167.318 82.46) (width 0.2) (layer "F.Cu") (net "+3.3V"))
 (segment (start 149.88 62) (end 149.88 65.5) (width 0.2) (layer "F.Cu") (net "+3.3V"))
 (segment (start 149.88 65.5) (end 142.830101 65.5) (width 0.2) (layer "F.Cu") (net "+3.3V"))
 (segment (start 167.318 82.46) (end 171 82.46) (width 0.2) (layer "F.Cu") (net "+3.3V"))
 (segment (start 154.901308 62) (end 153.236756 60.335448) (width 0.2) (layer "F.Cu") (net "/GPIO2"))
 (segment (start 180.85975 61.0045) (end 179.18475 59.3295) (width 0.2) (layer "F.Cu") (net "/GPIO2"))
 (segment (start 132.46 56.92) (end 149.821308 56.92) (width 0.2) (layer "F.Cu") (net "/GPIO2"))
 (segment (start 159.584714 59.3295) (end 156.914214 62) (width 0.2) (layer "F.Cu") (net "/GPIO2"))
 (segment (start 179.18475 59.3295) (end 159.584714 59.3295) (width 0.2) (layer "F.Cu") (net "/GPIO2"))
 (segment (start 149.821308 56.92) (end 153.236756 60.335448) (width 0.2) (layer "F.Cu") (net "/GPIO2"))
 (segment (start 156.914214 62) (end 154.901308 62) (width 0.2) (layer "F.Cu") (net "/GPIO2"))
 (segment (start 183.39975 61.0045) (end 181.32475 58.9295) (width 0.2) (layer "F.Cu") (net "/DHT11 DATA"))
 (segment (start 181.32475 58.9295) (end 158.5705 58.9295) (width 0.2) (layer "F.Cu") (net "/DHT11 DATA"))
 (segment (start 158.5705 58.9295) (end 156.5 61) (width 0.2) (layer "F.Cu") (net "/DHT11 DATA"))
 (segment (start 181.127542 63.0645) (end 181.5 63.436958) (width 0.2) (layer "F.Cu") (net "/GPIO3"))
 (segment (start 181.5 63.436958) (end 181.5 66) (width 0.2) (layer "F.Cu") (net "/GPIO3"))
 (segment (start 180.37975 63.0645) (end 181.127542 63.0645) (width 0.2) (layer "F.Cu") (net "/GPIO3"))
 (segment (start 181.3355 66.1645) (end 173.15975 66.1645) (width 0.2) (layer "F.Cu") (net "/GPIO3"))
 (segment (start 173.15975 66.1645) (end 160.86425 78.46) (width 0.2) (layer "F.Cu") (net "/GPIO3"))
 (segment (start 131.85 78.46) (end 160.86425 78.46) (width 0.2) (layer "F.Cu") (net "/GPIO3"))
 (segment (start 181.5 66) (end 181.3355 66.1645) (width 0.2) (layer "F.Cu") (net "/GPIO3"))
 (segment (start 178.31975 61.0045) (end 180.37975 63.0645) (width 0.2) (layer "F.Cu") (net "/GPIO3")))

